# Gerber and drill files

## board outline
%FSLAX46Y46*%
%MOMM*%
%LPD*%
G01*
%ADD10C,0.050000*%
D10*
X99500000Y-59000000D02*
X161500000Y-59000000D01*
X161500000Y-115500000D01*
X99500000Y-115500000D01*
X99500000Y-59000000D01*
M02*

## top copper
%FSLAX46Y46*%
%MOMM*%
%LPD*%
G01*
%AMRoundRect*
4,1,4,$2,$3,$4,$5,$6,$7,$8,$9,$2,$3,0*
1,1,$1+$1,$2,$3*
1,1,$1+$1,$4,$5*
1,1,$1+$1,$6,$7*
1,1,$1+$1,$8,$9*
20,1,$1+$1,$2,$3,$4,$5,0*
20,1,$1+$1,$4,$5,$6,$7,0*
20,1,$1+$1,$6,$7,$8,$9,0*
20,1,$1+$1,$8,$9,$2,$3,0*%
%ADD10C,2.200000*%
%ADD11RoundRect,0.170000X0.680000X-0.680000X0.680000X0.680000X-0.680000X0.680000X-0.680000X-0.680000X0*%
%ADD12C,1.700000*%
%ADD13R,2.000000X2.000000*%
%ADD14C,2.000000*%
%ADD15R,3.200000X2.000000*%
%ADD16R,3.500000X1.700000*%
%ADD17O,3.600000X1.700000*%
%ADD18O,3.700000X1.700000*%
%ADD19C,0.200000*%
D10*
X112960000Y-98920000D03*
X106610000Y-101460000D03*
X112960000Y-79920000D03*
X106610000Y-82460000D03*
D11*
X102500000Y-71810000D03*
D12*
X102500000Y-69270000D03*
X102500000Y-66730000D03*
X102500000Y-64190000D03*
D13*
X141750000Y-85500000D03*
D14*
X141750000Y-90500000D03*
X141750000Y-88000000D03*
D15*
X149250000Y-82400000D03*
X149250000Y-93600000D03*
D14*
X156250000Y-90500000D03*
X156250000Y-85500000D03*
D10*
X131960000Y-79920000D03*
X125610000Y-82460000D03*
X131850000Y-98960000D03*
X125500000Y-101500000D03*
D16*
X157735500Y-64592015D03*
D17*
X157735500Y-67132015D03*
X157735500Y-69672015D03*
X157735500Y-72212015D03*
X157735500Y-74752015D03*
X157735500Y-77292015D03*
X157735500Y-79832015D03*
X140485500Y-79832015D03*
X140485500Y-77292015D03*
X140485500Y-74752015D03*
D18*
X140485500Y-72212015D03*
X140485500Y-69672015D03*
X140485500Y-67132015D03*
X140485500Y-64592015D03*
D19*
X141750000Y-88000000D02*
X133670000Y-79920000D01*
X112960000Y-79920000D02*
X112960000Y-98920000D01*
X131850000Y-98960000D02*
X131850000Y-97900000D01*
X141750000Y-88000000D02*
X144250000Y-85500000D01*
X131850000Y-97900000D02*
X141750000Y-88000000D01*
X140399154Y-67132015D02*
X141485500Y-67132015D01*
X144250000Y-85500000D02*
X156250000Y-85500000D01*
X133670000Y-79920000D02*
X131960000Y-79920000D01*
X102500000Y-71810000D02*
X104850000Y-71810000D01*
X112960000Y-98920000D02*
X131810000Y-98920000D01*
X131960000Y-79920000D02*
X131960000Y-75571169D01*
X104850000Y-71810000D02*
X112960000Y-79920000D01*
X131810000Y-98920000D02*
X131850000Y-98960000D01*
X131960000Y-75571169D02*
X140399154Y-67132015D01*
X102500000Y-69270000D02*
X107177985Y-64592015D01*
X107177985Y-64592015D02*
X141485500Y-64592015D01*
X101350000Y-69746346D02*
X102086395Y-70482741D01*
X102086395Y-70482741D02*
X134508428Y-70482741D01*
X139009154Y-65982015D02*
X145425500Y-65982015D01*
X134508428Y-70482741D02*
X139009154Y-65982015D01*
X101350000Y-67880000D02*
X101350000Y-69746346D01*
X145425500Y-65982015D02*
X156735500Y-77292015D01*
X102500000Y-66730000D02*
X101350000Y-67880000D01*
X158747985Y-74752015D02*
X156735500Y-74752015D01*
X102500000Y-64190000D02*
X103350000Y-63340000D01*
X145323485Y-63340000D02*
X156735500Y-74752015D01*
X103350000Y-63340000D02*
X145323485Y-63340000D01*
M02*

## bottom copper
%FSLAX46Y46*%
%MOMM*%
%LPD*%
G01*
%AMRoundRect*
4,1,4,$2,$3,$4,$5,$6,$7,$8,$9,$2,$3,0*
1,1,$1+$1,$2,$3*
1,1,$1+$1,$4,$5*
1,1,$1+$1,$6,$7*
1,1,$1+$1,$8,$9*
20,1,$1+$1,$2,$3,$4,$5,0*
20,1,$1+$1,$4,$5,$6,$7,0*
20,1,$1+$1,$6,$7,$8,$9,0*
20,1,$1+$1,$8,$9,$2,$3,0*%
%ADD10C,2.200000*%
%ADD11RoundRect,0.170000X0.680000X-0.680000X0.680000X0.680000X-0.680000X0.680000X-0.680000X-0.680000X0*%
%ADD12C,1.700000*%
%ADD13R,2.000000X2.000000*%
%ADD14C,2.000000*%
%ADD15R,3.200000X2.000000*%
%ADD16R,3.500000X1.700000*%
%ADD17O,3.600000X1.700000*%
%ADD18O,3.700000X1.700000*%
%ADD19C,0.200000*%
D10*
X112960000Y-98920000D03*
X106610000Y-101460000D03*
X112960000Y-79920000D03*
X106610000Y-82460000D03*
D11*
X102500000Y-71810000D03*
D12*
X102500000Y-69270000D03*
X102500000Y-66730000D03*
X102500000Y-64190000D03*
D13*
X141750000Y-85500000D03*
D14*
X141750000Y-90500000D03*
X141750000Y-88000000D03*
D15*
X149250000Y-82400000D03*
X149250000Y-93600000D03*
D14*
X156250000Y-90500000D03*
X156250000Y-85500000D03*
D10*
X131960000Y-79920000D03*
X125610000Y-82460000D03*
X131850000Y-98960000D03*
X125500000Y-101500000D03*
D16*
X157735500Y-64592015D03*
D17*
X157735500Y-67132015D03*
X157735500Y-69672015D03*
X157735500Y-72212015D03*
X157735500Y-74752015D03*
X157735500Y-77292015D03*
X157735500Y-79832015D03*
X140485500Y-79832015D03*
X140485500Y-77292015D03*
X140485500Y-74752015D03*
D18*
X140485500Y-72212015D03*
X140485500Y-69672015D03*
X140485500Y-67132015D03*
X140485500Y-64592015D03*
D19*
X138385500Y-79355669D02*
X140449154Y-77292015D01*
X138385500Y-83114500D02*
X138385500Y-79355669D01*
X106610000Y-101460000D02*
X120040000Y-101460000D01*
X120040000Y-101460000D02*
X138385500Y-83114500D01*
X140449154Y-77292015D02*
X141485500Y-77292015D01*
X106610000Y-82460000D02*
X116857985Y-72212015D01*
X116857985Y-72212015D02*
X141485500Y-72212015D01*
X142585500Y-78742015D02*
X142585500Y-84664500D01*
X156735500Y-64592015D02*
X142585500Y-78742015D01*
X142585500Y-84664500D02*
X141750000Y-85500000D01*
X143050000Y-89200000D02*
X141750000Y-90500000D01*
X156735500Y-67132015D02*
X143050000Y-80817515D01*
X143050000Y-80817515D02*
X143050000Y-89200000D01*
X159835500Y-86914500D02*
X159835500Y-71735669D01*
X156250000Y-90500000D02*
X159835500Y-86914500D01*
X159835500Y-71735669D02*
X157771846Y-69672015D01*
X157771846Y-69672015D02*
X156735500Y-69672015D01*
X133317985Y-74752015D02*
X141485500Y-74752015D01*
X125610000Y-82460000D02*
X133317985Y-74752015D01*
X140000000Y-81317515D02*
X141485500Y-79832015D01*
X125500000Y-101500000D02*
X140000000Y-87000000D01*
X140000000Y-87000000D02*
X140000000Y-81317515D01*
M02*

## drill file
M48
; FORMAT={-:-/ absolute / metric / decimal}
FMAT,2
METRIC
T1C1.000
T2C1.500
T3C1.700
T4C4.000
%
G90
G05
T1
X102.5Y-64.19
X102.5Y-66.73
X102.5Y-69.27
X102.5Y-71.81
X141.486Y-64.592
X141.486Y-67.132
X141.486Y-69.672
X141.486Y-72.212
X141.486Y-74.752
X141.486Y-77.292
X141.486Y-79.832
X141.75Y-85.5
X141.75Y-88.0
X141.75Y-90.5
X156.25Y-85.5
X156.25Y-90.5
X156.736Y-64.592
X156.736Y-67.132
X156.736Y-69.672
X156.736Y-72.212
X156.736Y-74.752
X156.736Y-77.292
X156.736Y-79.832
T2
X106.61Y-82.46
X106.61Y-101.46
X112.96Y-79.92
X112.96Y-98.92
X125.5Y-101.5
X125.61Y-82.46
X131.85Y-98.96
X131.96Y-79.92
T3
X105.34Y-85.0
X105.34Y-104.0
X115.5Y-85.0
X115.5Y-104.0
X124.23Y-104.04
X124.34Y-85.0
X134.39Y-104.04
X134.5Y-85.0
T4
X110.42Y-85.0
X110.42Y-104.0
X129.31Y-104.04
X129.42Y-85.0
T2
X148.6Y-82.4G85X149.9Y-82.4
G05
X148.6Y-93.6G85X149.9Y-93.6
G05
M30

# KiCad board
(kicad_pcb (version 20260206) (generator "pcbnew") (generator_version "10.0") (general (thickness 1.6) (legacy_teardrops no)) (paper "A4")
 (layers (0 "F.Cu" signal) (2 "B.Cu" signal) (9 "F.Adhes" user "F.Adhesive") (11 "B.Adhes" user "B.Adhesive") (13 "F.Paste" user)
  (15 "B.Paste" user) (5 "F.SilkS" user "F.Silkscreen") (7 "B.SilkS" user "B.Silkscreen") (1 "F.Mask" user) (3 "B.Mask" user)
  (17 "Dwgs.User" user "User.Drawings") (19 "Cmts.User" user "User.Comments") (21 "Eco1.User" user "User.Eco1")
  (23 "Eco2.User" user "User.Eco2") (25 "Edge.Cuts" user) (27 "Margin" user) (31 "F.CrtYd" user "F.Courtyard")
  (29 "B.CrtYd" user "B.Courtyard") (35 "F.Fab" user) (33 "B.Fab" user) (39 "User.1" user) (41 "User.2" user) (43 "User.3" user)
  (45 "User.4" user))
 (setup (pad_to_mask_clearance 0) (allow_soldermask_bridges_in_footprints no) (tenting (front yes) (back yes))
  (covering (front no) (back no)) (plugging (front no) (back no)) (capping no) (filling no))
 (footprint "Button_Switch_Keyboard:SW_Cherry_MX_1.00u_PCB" (layer "F.Cu") (at 112.96 98.92)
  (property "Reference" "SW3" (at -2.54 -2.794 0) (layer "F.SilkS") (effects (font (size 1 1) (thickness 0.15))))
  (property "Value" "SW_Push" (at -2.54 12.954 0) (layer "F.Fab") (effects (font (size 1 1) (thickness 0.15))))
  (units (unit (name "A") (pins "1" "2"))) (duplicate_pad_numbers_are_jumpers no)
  (pad "" np_thru_hole circle (at -7.62 5.08) (size 1.7 1.7) (drill 1.7) (layers "*.Cu" "*.Mask"))
  (pad "" np_thru_hole circle (at -2.54 5.08) (size 4 4) (drill 4) (layers "*.Cu" "*.Mask"))
  (pad "" np_thru_hole circle (at 2.54 5.08) (size 1.7 1.7) (drill 1.7) (layers "*.Cu" "*.Mask"))
  (pad "1" thru_hole circle (at 0 0) (size 2.2 2.2) (drill 1.5) (layers "*.Cu" "*.Mask") (remove_unused_layers no) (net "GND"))
  (pad "2" thru_hole circle (at -6.35 2.54) (size 2.2 2.2) (drill 1.5) (layers "*.Cu" "*.Mask") (remove_unused_layers no)
   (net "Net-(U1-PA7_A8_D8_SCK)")))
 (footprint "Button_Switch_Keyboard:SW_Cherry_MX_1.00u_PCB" (layer "F.Cu") (at 112.96 79.92)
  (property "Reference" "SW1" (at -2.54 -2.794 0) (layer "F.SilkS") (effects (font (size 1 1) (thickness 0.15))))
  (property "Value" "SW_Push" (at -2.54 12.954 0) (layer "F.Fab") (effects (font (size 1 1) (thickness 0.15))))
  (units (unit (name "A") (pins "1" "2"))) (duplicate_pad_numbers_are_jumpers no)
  (pad "" np_thru_hole circle (at -7.62 5.08) (size 1.7 1.7) (drill 1.7) (layers "*.Cu" "*.Mask"))
  (pad "" np_thru_hole circle (at -2.54 5.08) (size 4 4) (drill 4) (layers "*.Cu" "*.Mask"))
  (pad "" np_thru_hole circle (at 2.54 5.08) (size 1.7 1.7) (drill 1.7) (layers "*.Cu" "*.Mask"))
  (pad "1" thru_hole circle (at 0 0) (size 2.2 2.2) (drill 1.5) (layers "*.Cu" "*.Mask") (remove_unused_layers no) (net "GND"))
  (pad "2" thru_hole circle (at -6.35 2.54) (size 2.2 2.2) (drill 1.5) (layers "*.Cu" "*.Mask") (remove_unused_layers no)
   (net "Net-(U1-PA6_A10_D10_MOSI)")))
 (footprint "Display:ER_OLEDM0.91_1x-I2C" (layer "F.Cu") (at 102.5 71.81 90)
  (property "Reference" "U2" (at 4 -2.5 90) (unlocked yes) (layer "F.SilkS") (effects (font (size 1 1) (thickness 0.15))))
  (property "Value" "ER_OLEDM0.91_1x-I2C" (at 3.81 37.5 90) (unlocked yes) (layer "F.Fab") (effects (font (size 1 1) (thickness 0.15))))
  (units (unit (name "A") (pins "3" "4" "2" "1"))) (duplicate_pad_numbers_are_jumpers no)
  (pad "1" thru_hole roundrect (at 0 0 90) (size 1.7 1.7) (drill 1) (layers "*.Cu" "*.Mask") (remove_unused_layers no)
   (roundrect_rratio 0.1) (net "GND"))
  (pad "2" thru_hole circle (at 2.54 0 90) (size 1.7 1.7) (drill 1) (layers "*.Cu" "*.Mask") (remove_unused_layers no) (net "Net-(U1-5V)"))
  (pad "3" thru_hole circle (at 5.08 0 90) (size 1.7 1.7) (drill 1) (layers "*.Cu" "*.Mask") (remove_unused_layers no)
   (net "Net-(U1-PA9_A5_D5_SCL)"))
  (pad "4" thru_hole circle (at 7.62 0 90) (size 1.7 1.7) (drill 1) (layers "*.Cu" "*.Mask") (remove_unused_layers no)
   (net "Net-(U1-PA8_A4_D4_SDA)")))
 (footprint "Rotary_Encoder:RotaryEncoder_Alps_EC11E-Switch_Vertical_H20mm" (layer "F.Cu") (at 141.75 85.5)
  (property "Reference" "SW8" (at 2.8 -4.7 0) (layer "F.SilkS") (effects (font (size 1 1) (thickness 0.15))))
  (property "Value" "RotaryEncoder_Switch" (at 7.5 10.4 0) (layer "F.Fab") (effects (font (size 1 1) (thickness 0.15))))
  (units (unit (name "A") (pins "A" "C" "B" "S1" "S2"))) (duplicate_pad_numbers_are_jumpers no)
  (pad "A" thru_hole rect (at 0 0) (size 2 2) (drill 1) (layers "*.Cu" "*.Mask") (remove_unused_layers no) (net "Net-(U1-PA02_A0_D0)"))
  (pad "B" thru_hole circle (at 0 5) (size 2 2) (drill 1) (layers "*.Cu" "*.Mask") (remove_unused_layers no) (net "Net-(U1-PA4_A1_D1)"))
  (pad "C" thru_hole circle (at 0 2.5) (size 2 2) (drill 1) (layers "*.Cu" "*.Mask") (remove_unused_layers no) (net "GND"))
  (pad "MP" thru_hole rect (at 7.5 -3.1) (size 3.2 2) (drill oval 2.8 1.5) (layers "*.Cu" "*.Mask") (remove_unused_layers no))
  (pad "MP" thru_hole rect (at 7.5 8.1) (size 3.2 2) (drill oval 2.8 1.5) (layers "*.Cu" "*.Mask") (remove_unused_layers no))
  (pad "S1" thru_hole circle (at 14.5 5) (size 2 2) (drill 1) (layers "*.Cu" "*.Mask") (remove_unused_layers no) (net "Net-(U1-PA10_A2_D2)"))
  (pad "S2" thru_hole circle (at 14.5 0) (size 2 2) (drill 1) (layers "*.Cu" "*.Mask") (remove_unused_layers no) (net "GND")))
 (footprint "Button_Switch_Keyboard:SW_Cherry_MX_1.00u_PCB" (layer "F.Cu") (at 131.96 79.92)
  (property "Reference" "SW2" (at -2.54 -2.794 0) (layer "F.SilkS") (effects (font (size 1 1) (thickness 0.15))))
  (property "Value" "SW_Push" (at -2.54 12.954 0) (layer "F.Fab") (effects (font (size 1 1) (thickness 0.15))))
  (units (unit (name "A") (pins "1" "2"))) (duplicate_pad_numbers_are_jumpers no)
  (pad "" np_thru_hole circle (at -7.62 5.08) (size 1.7 1.7) (drill 1.7) (layers "*.Cu" "*.Mask"))
  (pad "" np_thru_hole circle (at -2.54 5.08) (size 4 4) (drill 4) (layers "*.Cu" "*.Mask"))
  (pad "" np_thru_hole circle (at 2.54 5.08) (size 1.7 1.7) (drill 1.7) (layers "*.Cu" "*.Mask"))
  (pad "1" thru_hole circle (at 0 0) (size 2.2 2.2) (drill 1.5) (layers "*.Cu" "*.Mask") (remove_unused_layers no) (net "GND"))
  (pad "2" thru_hole circle (at -6.35 2.54) (size 2.2 2.2) (drill 1.5) (layers "*.Cu" "*.Mask") (remove_unused_layers no)
   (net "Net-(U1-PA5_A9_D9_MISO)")))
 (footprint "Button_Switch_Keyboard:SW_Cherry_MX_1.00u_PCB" (layer "F.Cu") (at 131.85 98.96)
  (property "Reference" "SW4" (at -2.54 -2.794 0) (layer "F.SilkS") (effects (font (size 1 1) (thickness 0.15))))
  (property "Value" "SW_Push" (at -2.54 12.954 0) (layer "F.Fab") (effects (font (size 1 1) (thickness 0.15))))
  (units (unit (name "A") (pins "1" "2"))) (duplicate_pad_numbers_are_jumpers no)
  (pad "" np_thru_hole circle (at -7.62 5.08) (size 1.7 1.7) (drill 1.7) (layers "*.Cu" "*.Mask"))
  (pad "" np_thru_hole circle (at -2.54 5.08) (size 4 4) (drill 4) (layers "*.Cu" "*.Mask"))
  (pad "" np_thru_hole circle (at 2.54 5.08) (size 1.7 1.7) (drill 1.7) (layers "*.Cu" "*.Mask"))
  (pad "1" thru_hole circle (at 0 0) (size 2.2 2.2) (drill 1.5) (layers "*.Cu" "*.Mask") (remove_unused_layers no) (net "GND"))
  (pad "2" thru_hole circle (at -6.35 2.54) (size 2.2 2.2) (drill 1.5) (layers "*.Cu" "*.Mask") (remove_unused_layers no)
   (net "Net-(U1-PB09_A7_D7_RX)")))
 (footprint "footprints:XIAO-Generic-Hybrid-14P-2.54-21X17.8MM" (layer "B.Cu") (at 149.1105 72.212015 180)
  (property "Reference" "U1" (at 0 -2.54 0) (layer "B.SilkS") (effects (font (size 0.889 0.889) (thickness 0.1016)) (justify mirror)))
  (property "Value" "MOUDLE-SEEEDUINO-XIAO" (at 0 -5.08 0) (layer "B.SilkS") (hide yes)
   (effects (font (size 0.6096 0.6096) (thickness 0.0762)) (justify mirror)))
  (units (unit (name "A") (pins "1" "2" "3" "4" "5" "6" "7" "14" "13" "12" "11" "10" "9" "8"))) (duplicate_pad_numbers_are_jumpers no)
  (pad "1" thru_hole rect (at -7.625 7.62 180) (size 3.5 1.7) (drill 1 (offset -1 0)) (layers "*.Cu" "*.Mask") (remove_unused_layers no)
   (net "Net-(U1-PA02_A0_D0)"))
  (pad "2" thru_hole oval (at -7.625 5.08 180) (size 3.6 1.7) (drill 1 (offset -1 0)) (layers "*.Cu" "*.Mask") (remove_unused_layers no)
   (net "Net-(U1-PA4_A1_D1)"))
  (pad "3" thru_hole oval (at -7.625 2.54 180) (size 3.6 1.7) (drill 1 (offset -1 0)) (layers "*.Cu" "*.Mask") (remove_unused_layers no)
   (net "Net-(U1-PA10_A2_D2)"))
  (pad "4" thru_hole oval (at -7.625 0 180) (size 3.6 1.7) (drill 1 (offset -1 0)) (layers "*.Cu" "*.Mask") (remove_unused_layers no)
   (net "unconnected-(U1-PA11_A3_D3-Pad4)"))
  (pad "5" thru_hole oval (at -7.625 -2.54 180) (size 3.6 1.7) (drill 1 (offset -1 0)) (layers "*.Cu" "*.Mask") (remove_unused_layers no)
   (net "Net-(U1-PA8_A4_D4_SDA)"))
  (pad "6" thru_hole oval (at -7.625 -5.08) (size 3.6 1.7) (drill 1 (offset 1 0)) (layers "*.Cu" "*.Mask") (remove_unused_layers no)
   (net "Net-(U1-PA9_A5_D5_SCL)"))
  (pad "7" thru_hole oval (at -7.625 -7.62 180) (size 3.6 1.7) (drill 1 (offset -1 0)) (layers "*.Cu" "*.Mask") (remove_unused_layers no)
   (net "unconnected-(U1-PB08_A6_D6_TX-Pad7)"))
  (pad "8" thru_hole oval (at 7.625 -7.62 180) (size 3.6 1.7) (drill 1 (offset 1 0)) (layers "*.Cu" "*.Mask") (remove_unused_layers no)
   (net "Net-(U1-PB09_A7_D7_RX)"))
  (pad "9" thru_hole oval (at 7.625 -5.08 180) (size 3.6 1.7) (drill 1 (offset 1 0)) (layers "*.Cu" "*.Mask") (remove_unused_layers no)
   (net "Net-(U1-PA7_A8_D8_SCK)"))
  (pad "10" thru_hole oval (at 7.625 -2.54 180) (size 3.6 1.7) (drill 1 (offset 1 0)) (layers "*.Cu" "*.Mask") (remove_unused_layers no)
   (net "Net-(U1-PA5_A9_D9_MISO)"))
  (pad "11" thru_hole oval (at 7.625 0 180) (size 3.7 1.7) (drill 1 (offset 1 0)) (layers "*.Cu" "*.Mask") (remove_unused_layers no)
   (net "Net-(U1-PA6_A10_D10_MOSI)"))
  (pad "12" thru_hole oval (at 7.625 2.54 180) (size 3.7 1.7) (drill 1 (offset 1 0)) (layers "*.Cu" "*.Mask") (remove_unused_layers no)
   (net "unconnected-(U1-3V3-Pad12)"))
  (pad "13" thru_hole oval (at 7.625 5.08 180) (size 3.7 1.7) (drill 1 (offset 1 0)) (layers "*.Cu" "*.Mask") (remove_unused_layers no)
   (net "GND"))
  (pad "14" thru_hole oval (at 7.625 7.62 180) (size 3.7 1.7) (drill 1 (offset 1 0)) (layers "*.Cu" "*.Mask") (remove_unused_layers no)
   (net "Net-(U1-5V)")))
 (gr_rect (start 99.5 59) (end 161.5 115.5) (stroke (width 0.05) (type default)) (fill no) (layer "Edge.Cuts"))
 (segment (start 141.75 88) (end 133.67 79.92) (width 0.2) (layer "F.Cu") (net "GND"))
 (segment (start 112.96 79.92) (end 112.96 98.92) (width 0.2) (layer "F.Cu") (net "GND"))
 (segment (start 131.85 98.96) (end 131.85 97.9) (width 0.2) (layer "F.Cu") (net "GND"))
 (segment (start 141.75 88) (end 144.25 85.5) (width 0.2) (layer "F.Cu") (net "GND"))
 (segment (start 131.85 97.9) (end 141.75 88) (width 0.2) (layer "F.Cu") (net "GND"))
 (segment (start 140.399154 67.132015) (end 141.4855 67.132015) (width 0.2) (layer "F.Cu") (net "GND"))
 (segment (start 144.25 85.5) (end 156.25 85.5) (width 0.2) (layer "F.Cu") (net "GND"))
 (segment (start 133.67 79.92) (end 131.96 79.92) (width 0.2) (layer "F.Cu") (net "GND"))
 (segment (start 102.5 71.81) (end 104.85 71.81) (width 0.2) (layer "F.Cu") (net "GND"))
 (segment (start 112.96 98.92) (end 131.81 98.92) (width 0.2) (layer "F.Cu") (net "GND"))
 (segment (start 131.96 79.92) (end 131.96 75.571169) (width 0.2) (layer "F.Cu") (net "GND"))
 (segment (start 104.85 71.81) (end 112.96 79.92) (width 0.2) (layer "F.Cu") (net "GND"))
 (segment (start 131.81 98.92) (end 131.85 98.96) (width 0.2) (layer "F.Cu") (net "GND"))
 (segment (start 131.96 75.571169) (end 140.399154 67.132015) (width 0.2) (layer "F.Cu") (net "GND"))
 (segment (start 138.3855 79.355669) (end 140.449154 77.292015) (width 0.2) (layer "B.Cu") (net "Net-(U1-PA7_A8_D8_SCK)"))
 (segment (start 138.3855 83.1145) (end 138.3855 79.355669) (width 0.2) (layer "B.Cu") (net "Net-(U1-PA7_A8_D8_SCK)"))
 (segment (start 106.61 101.46) (end 120.04 101.46) (width 0.2) (layer "B.Cu") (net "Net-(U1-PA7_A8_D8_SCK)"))
 (segment (start 120.04 101.46) (end 138.3855 83.1145) (width 0.2) (layer "B.Cu") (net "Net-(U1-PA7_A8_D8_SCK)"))
 (segment (start 140.449154 77.292015) (end 141.4855 77.292015) (width 0.2) (layer "B.Cu") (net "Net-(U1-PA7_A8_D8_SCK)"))
 (segment (start 106.61 82.46) (end 116.857985 72.212015) (width 0.2) (layer "B.Cu") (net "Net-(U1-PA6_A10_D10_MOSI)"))
 (segment (start 116.857985 72.212015) (end 141.4855 72.212015) (width 0.2) (layer "B.Cu") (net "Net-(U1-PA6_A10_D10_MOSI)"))
 (segment (start 102.5 69.27) (end 107.177985 64.592015) (width 0.2) (layer "F.Cu") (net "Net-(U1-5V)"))
 (segment (start 107.177985 64.592015) (end 141.4855 64.592015) (width 0.2) (layer "F.Cu") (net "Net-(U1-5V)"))
 (segment (start 101.35 69.746346) (end 102.086395 70.482741) (width 0.2) (layer "F.Cu") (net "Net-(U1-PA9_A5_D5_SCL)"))
 (segment (start 102.086395 70.482741) (end 134.508428 70.482741) (width 0.2) (layer "F.Cu") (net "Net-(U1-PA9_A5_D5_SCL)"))
 (segment (start 139.009154 65.982015) (end 145.4255 65.982015) (width 0.2) (layer "F.Cu") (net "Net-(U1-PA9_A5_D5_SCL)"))
 (segment (start 134.508428 70.482741) (end 139.009154 65.982015) (width 0.2) (layer "F.Cu") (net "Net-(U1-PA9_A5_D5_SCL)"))
 (segment (start 101.35 67.88) (end 101.35 69.746346) (width 0.2) (layer "F.Cu") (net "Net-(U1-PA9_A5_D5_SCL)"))
 (segment (start 145.4255 65.982015) (end 156.7355 77.292015) (width 0.2) (layer "F.Cu") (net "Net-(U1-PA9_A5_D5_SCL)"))
 (segment (start 102.5 66.73) (end 101.35 67.88) (width 0.2) (layer "F.Cu") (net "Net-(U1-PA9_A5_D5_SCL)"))
 (segment (start 158.747985 74.752015) (end 156.7355 74.752015) (width 0.2) (layer "F.Cu") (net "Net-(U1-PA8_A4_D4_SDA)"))
 (segment (start 102.5 64.19) (end 103.35 63.34) (width 0.2) (layer "F.Cu") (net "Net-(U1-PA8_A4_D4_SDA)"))
 (segment (start 145.323485 63.34) (end 156.7355 74.752015) (width 0.2) (layer "F.Cu") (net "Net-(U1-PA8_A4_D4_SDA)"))
 (segment (start 103.35 63.34) (end 145.323485 63.34) (width 0.2) (layer "F.Cu") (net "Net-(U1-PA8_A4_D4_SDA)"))
 (segment (start 142.5855 78.742015) (end 142.5855 84.6645) (width 0.2) (layer "B.Cu") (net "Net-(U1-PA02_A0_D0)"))
 (segment (start 156.7355 64.592015) (end 142.5855 78.742015) (width 0.2) (layer "B.Cu") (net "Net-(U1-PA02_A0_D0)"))
 (segment (start 142.5855 84.6645) (end 141.75 85.5) (width 0.2) (layer "B.Cu") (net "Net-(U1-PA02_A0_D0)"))
 (segment (start 143.05 89.2) (end 141.75 90.5) (width 0.2) (layer "B.Cu") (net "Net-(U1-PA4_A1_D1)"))
 (segment (start 156.7355 67.132015) (end 143.05 80.817515) (width 0.2) (layer "B.Cu") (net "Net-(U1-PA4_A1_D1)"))
 (segment (start 143.05 80.817515) (end 143.05 89.2) (width 0.2) (layer "B.Cu") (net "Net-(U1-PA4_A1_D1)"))
 (segment (start 159.8355 86.9145) (end 159.8355 71.735669) (width 0.2) (layer "B.Cu") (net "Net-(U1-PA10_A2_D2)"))
 (segment (start 156.25 90.5) (end 159.8355 86.9145) (width 0.2) (layer "B.Cu") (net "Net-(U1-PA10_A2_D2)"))
 (segment (start 159.8355 71.735669) (end 157.771846 69.672015) (width 0.2) (layer "B.Cu") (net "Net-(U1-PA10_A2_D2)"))
 (segment (start 157.771846 69.672015) (end 156.7355 69.672015) (width 0.2) (layer "B.Cu") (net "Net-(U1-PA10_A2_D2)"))
 (segment (start 133.317985 74.752015) (end 141.4855 74.752015) (width 0.2) (layer "B.Cu") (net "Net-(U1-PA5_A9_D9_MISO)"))
 (segment (start 125.61 82.46) (end 133.317985 74.752015) (width 0.2) (layer "B.Cu") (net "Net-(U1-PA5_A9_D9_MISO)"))
 (segment (start 140 81.317515) (end 141.4855 79.832015) (width 0.2) (layer "B.Cu") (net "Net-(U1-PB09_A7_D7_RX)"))
 (segment (start 125.5 101.5) (end 140 87) (width 0.2) (layer "B.Cu") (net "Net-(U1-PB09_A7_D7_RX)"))
 (segment (start 140 87) (end 140 81.317515) (width 0.2) (layer "B.Cu") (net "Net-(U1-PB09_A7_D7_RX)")))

